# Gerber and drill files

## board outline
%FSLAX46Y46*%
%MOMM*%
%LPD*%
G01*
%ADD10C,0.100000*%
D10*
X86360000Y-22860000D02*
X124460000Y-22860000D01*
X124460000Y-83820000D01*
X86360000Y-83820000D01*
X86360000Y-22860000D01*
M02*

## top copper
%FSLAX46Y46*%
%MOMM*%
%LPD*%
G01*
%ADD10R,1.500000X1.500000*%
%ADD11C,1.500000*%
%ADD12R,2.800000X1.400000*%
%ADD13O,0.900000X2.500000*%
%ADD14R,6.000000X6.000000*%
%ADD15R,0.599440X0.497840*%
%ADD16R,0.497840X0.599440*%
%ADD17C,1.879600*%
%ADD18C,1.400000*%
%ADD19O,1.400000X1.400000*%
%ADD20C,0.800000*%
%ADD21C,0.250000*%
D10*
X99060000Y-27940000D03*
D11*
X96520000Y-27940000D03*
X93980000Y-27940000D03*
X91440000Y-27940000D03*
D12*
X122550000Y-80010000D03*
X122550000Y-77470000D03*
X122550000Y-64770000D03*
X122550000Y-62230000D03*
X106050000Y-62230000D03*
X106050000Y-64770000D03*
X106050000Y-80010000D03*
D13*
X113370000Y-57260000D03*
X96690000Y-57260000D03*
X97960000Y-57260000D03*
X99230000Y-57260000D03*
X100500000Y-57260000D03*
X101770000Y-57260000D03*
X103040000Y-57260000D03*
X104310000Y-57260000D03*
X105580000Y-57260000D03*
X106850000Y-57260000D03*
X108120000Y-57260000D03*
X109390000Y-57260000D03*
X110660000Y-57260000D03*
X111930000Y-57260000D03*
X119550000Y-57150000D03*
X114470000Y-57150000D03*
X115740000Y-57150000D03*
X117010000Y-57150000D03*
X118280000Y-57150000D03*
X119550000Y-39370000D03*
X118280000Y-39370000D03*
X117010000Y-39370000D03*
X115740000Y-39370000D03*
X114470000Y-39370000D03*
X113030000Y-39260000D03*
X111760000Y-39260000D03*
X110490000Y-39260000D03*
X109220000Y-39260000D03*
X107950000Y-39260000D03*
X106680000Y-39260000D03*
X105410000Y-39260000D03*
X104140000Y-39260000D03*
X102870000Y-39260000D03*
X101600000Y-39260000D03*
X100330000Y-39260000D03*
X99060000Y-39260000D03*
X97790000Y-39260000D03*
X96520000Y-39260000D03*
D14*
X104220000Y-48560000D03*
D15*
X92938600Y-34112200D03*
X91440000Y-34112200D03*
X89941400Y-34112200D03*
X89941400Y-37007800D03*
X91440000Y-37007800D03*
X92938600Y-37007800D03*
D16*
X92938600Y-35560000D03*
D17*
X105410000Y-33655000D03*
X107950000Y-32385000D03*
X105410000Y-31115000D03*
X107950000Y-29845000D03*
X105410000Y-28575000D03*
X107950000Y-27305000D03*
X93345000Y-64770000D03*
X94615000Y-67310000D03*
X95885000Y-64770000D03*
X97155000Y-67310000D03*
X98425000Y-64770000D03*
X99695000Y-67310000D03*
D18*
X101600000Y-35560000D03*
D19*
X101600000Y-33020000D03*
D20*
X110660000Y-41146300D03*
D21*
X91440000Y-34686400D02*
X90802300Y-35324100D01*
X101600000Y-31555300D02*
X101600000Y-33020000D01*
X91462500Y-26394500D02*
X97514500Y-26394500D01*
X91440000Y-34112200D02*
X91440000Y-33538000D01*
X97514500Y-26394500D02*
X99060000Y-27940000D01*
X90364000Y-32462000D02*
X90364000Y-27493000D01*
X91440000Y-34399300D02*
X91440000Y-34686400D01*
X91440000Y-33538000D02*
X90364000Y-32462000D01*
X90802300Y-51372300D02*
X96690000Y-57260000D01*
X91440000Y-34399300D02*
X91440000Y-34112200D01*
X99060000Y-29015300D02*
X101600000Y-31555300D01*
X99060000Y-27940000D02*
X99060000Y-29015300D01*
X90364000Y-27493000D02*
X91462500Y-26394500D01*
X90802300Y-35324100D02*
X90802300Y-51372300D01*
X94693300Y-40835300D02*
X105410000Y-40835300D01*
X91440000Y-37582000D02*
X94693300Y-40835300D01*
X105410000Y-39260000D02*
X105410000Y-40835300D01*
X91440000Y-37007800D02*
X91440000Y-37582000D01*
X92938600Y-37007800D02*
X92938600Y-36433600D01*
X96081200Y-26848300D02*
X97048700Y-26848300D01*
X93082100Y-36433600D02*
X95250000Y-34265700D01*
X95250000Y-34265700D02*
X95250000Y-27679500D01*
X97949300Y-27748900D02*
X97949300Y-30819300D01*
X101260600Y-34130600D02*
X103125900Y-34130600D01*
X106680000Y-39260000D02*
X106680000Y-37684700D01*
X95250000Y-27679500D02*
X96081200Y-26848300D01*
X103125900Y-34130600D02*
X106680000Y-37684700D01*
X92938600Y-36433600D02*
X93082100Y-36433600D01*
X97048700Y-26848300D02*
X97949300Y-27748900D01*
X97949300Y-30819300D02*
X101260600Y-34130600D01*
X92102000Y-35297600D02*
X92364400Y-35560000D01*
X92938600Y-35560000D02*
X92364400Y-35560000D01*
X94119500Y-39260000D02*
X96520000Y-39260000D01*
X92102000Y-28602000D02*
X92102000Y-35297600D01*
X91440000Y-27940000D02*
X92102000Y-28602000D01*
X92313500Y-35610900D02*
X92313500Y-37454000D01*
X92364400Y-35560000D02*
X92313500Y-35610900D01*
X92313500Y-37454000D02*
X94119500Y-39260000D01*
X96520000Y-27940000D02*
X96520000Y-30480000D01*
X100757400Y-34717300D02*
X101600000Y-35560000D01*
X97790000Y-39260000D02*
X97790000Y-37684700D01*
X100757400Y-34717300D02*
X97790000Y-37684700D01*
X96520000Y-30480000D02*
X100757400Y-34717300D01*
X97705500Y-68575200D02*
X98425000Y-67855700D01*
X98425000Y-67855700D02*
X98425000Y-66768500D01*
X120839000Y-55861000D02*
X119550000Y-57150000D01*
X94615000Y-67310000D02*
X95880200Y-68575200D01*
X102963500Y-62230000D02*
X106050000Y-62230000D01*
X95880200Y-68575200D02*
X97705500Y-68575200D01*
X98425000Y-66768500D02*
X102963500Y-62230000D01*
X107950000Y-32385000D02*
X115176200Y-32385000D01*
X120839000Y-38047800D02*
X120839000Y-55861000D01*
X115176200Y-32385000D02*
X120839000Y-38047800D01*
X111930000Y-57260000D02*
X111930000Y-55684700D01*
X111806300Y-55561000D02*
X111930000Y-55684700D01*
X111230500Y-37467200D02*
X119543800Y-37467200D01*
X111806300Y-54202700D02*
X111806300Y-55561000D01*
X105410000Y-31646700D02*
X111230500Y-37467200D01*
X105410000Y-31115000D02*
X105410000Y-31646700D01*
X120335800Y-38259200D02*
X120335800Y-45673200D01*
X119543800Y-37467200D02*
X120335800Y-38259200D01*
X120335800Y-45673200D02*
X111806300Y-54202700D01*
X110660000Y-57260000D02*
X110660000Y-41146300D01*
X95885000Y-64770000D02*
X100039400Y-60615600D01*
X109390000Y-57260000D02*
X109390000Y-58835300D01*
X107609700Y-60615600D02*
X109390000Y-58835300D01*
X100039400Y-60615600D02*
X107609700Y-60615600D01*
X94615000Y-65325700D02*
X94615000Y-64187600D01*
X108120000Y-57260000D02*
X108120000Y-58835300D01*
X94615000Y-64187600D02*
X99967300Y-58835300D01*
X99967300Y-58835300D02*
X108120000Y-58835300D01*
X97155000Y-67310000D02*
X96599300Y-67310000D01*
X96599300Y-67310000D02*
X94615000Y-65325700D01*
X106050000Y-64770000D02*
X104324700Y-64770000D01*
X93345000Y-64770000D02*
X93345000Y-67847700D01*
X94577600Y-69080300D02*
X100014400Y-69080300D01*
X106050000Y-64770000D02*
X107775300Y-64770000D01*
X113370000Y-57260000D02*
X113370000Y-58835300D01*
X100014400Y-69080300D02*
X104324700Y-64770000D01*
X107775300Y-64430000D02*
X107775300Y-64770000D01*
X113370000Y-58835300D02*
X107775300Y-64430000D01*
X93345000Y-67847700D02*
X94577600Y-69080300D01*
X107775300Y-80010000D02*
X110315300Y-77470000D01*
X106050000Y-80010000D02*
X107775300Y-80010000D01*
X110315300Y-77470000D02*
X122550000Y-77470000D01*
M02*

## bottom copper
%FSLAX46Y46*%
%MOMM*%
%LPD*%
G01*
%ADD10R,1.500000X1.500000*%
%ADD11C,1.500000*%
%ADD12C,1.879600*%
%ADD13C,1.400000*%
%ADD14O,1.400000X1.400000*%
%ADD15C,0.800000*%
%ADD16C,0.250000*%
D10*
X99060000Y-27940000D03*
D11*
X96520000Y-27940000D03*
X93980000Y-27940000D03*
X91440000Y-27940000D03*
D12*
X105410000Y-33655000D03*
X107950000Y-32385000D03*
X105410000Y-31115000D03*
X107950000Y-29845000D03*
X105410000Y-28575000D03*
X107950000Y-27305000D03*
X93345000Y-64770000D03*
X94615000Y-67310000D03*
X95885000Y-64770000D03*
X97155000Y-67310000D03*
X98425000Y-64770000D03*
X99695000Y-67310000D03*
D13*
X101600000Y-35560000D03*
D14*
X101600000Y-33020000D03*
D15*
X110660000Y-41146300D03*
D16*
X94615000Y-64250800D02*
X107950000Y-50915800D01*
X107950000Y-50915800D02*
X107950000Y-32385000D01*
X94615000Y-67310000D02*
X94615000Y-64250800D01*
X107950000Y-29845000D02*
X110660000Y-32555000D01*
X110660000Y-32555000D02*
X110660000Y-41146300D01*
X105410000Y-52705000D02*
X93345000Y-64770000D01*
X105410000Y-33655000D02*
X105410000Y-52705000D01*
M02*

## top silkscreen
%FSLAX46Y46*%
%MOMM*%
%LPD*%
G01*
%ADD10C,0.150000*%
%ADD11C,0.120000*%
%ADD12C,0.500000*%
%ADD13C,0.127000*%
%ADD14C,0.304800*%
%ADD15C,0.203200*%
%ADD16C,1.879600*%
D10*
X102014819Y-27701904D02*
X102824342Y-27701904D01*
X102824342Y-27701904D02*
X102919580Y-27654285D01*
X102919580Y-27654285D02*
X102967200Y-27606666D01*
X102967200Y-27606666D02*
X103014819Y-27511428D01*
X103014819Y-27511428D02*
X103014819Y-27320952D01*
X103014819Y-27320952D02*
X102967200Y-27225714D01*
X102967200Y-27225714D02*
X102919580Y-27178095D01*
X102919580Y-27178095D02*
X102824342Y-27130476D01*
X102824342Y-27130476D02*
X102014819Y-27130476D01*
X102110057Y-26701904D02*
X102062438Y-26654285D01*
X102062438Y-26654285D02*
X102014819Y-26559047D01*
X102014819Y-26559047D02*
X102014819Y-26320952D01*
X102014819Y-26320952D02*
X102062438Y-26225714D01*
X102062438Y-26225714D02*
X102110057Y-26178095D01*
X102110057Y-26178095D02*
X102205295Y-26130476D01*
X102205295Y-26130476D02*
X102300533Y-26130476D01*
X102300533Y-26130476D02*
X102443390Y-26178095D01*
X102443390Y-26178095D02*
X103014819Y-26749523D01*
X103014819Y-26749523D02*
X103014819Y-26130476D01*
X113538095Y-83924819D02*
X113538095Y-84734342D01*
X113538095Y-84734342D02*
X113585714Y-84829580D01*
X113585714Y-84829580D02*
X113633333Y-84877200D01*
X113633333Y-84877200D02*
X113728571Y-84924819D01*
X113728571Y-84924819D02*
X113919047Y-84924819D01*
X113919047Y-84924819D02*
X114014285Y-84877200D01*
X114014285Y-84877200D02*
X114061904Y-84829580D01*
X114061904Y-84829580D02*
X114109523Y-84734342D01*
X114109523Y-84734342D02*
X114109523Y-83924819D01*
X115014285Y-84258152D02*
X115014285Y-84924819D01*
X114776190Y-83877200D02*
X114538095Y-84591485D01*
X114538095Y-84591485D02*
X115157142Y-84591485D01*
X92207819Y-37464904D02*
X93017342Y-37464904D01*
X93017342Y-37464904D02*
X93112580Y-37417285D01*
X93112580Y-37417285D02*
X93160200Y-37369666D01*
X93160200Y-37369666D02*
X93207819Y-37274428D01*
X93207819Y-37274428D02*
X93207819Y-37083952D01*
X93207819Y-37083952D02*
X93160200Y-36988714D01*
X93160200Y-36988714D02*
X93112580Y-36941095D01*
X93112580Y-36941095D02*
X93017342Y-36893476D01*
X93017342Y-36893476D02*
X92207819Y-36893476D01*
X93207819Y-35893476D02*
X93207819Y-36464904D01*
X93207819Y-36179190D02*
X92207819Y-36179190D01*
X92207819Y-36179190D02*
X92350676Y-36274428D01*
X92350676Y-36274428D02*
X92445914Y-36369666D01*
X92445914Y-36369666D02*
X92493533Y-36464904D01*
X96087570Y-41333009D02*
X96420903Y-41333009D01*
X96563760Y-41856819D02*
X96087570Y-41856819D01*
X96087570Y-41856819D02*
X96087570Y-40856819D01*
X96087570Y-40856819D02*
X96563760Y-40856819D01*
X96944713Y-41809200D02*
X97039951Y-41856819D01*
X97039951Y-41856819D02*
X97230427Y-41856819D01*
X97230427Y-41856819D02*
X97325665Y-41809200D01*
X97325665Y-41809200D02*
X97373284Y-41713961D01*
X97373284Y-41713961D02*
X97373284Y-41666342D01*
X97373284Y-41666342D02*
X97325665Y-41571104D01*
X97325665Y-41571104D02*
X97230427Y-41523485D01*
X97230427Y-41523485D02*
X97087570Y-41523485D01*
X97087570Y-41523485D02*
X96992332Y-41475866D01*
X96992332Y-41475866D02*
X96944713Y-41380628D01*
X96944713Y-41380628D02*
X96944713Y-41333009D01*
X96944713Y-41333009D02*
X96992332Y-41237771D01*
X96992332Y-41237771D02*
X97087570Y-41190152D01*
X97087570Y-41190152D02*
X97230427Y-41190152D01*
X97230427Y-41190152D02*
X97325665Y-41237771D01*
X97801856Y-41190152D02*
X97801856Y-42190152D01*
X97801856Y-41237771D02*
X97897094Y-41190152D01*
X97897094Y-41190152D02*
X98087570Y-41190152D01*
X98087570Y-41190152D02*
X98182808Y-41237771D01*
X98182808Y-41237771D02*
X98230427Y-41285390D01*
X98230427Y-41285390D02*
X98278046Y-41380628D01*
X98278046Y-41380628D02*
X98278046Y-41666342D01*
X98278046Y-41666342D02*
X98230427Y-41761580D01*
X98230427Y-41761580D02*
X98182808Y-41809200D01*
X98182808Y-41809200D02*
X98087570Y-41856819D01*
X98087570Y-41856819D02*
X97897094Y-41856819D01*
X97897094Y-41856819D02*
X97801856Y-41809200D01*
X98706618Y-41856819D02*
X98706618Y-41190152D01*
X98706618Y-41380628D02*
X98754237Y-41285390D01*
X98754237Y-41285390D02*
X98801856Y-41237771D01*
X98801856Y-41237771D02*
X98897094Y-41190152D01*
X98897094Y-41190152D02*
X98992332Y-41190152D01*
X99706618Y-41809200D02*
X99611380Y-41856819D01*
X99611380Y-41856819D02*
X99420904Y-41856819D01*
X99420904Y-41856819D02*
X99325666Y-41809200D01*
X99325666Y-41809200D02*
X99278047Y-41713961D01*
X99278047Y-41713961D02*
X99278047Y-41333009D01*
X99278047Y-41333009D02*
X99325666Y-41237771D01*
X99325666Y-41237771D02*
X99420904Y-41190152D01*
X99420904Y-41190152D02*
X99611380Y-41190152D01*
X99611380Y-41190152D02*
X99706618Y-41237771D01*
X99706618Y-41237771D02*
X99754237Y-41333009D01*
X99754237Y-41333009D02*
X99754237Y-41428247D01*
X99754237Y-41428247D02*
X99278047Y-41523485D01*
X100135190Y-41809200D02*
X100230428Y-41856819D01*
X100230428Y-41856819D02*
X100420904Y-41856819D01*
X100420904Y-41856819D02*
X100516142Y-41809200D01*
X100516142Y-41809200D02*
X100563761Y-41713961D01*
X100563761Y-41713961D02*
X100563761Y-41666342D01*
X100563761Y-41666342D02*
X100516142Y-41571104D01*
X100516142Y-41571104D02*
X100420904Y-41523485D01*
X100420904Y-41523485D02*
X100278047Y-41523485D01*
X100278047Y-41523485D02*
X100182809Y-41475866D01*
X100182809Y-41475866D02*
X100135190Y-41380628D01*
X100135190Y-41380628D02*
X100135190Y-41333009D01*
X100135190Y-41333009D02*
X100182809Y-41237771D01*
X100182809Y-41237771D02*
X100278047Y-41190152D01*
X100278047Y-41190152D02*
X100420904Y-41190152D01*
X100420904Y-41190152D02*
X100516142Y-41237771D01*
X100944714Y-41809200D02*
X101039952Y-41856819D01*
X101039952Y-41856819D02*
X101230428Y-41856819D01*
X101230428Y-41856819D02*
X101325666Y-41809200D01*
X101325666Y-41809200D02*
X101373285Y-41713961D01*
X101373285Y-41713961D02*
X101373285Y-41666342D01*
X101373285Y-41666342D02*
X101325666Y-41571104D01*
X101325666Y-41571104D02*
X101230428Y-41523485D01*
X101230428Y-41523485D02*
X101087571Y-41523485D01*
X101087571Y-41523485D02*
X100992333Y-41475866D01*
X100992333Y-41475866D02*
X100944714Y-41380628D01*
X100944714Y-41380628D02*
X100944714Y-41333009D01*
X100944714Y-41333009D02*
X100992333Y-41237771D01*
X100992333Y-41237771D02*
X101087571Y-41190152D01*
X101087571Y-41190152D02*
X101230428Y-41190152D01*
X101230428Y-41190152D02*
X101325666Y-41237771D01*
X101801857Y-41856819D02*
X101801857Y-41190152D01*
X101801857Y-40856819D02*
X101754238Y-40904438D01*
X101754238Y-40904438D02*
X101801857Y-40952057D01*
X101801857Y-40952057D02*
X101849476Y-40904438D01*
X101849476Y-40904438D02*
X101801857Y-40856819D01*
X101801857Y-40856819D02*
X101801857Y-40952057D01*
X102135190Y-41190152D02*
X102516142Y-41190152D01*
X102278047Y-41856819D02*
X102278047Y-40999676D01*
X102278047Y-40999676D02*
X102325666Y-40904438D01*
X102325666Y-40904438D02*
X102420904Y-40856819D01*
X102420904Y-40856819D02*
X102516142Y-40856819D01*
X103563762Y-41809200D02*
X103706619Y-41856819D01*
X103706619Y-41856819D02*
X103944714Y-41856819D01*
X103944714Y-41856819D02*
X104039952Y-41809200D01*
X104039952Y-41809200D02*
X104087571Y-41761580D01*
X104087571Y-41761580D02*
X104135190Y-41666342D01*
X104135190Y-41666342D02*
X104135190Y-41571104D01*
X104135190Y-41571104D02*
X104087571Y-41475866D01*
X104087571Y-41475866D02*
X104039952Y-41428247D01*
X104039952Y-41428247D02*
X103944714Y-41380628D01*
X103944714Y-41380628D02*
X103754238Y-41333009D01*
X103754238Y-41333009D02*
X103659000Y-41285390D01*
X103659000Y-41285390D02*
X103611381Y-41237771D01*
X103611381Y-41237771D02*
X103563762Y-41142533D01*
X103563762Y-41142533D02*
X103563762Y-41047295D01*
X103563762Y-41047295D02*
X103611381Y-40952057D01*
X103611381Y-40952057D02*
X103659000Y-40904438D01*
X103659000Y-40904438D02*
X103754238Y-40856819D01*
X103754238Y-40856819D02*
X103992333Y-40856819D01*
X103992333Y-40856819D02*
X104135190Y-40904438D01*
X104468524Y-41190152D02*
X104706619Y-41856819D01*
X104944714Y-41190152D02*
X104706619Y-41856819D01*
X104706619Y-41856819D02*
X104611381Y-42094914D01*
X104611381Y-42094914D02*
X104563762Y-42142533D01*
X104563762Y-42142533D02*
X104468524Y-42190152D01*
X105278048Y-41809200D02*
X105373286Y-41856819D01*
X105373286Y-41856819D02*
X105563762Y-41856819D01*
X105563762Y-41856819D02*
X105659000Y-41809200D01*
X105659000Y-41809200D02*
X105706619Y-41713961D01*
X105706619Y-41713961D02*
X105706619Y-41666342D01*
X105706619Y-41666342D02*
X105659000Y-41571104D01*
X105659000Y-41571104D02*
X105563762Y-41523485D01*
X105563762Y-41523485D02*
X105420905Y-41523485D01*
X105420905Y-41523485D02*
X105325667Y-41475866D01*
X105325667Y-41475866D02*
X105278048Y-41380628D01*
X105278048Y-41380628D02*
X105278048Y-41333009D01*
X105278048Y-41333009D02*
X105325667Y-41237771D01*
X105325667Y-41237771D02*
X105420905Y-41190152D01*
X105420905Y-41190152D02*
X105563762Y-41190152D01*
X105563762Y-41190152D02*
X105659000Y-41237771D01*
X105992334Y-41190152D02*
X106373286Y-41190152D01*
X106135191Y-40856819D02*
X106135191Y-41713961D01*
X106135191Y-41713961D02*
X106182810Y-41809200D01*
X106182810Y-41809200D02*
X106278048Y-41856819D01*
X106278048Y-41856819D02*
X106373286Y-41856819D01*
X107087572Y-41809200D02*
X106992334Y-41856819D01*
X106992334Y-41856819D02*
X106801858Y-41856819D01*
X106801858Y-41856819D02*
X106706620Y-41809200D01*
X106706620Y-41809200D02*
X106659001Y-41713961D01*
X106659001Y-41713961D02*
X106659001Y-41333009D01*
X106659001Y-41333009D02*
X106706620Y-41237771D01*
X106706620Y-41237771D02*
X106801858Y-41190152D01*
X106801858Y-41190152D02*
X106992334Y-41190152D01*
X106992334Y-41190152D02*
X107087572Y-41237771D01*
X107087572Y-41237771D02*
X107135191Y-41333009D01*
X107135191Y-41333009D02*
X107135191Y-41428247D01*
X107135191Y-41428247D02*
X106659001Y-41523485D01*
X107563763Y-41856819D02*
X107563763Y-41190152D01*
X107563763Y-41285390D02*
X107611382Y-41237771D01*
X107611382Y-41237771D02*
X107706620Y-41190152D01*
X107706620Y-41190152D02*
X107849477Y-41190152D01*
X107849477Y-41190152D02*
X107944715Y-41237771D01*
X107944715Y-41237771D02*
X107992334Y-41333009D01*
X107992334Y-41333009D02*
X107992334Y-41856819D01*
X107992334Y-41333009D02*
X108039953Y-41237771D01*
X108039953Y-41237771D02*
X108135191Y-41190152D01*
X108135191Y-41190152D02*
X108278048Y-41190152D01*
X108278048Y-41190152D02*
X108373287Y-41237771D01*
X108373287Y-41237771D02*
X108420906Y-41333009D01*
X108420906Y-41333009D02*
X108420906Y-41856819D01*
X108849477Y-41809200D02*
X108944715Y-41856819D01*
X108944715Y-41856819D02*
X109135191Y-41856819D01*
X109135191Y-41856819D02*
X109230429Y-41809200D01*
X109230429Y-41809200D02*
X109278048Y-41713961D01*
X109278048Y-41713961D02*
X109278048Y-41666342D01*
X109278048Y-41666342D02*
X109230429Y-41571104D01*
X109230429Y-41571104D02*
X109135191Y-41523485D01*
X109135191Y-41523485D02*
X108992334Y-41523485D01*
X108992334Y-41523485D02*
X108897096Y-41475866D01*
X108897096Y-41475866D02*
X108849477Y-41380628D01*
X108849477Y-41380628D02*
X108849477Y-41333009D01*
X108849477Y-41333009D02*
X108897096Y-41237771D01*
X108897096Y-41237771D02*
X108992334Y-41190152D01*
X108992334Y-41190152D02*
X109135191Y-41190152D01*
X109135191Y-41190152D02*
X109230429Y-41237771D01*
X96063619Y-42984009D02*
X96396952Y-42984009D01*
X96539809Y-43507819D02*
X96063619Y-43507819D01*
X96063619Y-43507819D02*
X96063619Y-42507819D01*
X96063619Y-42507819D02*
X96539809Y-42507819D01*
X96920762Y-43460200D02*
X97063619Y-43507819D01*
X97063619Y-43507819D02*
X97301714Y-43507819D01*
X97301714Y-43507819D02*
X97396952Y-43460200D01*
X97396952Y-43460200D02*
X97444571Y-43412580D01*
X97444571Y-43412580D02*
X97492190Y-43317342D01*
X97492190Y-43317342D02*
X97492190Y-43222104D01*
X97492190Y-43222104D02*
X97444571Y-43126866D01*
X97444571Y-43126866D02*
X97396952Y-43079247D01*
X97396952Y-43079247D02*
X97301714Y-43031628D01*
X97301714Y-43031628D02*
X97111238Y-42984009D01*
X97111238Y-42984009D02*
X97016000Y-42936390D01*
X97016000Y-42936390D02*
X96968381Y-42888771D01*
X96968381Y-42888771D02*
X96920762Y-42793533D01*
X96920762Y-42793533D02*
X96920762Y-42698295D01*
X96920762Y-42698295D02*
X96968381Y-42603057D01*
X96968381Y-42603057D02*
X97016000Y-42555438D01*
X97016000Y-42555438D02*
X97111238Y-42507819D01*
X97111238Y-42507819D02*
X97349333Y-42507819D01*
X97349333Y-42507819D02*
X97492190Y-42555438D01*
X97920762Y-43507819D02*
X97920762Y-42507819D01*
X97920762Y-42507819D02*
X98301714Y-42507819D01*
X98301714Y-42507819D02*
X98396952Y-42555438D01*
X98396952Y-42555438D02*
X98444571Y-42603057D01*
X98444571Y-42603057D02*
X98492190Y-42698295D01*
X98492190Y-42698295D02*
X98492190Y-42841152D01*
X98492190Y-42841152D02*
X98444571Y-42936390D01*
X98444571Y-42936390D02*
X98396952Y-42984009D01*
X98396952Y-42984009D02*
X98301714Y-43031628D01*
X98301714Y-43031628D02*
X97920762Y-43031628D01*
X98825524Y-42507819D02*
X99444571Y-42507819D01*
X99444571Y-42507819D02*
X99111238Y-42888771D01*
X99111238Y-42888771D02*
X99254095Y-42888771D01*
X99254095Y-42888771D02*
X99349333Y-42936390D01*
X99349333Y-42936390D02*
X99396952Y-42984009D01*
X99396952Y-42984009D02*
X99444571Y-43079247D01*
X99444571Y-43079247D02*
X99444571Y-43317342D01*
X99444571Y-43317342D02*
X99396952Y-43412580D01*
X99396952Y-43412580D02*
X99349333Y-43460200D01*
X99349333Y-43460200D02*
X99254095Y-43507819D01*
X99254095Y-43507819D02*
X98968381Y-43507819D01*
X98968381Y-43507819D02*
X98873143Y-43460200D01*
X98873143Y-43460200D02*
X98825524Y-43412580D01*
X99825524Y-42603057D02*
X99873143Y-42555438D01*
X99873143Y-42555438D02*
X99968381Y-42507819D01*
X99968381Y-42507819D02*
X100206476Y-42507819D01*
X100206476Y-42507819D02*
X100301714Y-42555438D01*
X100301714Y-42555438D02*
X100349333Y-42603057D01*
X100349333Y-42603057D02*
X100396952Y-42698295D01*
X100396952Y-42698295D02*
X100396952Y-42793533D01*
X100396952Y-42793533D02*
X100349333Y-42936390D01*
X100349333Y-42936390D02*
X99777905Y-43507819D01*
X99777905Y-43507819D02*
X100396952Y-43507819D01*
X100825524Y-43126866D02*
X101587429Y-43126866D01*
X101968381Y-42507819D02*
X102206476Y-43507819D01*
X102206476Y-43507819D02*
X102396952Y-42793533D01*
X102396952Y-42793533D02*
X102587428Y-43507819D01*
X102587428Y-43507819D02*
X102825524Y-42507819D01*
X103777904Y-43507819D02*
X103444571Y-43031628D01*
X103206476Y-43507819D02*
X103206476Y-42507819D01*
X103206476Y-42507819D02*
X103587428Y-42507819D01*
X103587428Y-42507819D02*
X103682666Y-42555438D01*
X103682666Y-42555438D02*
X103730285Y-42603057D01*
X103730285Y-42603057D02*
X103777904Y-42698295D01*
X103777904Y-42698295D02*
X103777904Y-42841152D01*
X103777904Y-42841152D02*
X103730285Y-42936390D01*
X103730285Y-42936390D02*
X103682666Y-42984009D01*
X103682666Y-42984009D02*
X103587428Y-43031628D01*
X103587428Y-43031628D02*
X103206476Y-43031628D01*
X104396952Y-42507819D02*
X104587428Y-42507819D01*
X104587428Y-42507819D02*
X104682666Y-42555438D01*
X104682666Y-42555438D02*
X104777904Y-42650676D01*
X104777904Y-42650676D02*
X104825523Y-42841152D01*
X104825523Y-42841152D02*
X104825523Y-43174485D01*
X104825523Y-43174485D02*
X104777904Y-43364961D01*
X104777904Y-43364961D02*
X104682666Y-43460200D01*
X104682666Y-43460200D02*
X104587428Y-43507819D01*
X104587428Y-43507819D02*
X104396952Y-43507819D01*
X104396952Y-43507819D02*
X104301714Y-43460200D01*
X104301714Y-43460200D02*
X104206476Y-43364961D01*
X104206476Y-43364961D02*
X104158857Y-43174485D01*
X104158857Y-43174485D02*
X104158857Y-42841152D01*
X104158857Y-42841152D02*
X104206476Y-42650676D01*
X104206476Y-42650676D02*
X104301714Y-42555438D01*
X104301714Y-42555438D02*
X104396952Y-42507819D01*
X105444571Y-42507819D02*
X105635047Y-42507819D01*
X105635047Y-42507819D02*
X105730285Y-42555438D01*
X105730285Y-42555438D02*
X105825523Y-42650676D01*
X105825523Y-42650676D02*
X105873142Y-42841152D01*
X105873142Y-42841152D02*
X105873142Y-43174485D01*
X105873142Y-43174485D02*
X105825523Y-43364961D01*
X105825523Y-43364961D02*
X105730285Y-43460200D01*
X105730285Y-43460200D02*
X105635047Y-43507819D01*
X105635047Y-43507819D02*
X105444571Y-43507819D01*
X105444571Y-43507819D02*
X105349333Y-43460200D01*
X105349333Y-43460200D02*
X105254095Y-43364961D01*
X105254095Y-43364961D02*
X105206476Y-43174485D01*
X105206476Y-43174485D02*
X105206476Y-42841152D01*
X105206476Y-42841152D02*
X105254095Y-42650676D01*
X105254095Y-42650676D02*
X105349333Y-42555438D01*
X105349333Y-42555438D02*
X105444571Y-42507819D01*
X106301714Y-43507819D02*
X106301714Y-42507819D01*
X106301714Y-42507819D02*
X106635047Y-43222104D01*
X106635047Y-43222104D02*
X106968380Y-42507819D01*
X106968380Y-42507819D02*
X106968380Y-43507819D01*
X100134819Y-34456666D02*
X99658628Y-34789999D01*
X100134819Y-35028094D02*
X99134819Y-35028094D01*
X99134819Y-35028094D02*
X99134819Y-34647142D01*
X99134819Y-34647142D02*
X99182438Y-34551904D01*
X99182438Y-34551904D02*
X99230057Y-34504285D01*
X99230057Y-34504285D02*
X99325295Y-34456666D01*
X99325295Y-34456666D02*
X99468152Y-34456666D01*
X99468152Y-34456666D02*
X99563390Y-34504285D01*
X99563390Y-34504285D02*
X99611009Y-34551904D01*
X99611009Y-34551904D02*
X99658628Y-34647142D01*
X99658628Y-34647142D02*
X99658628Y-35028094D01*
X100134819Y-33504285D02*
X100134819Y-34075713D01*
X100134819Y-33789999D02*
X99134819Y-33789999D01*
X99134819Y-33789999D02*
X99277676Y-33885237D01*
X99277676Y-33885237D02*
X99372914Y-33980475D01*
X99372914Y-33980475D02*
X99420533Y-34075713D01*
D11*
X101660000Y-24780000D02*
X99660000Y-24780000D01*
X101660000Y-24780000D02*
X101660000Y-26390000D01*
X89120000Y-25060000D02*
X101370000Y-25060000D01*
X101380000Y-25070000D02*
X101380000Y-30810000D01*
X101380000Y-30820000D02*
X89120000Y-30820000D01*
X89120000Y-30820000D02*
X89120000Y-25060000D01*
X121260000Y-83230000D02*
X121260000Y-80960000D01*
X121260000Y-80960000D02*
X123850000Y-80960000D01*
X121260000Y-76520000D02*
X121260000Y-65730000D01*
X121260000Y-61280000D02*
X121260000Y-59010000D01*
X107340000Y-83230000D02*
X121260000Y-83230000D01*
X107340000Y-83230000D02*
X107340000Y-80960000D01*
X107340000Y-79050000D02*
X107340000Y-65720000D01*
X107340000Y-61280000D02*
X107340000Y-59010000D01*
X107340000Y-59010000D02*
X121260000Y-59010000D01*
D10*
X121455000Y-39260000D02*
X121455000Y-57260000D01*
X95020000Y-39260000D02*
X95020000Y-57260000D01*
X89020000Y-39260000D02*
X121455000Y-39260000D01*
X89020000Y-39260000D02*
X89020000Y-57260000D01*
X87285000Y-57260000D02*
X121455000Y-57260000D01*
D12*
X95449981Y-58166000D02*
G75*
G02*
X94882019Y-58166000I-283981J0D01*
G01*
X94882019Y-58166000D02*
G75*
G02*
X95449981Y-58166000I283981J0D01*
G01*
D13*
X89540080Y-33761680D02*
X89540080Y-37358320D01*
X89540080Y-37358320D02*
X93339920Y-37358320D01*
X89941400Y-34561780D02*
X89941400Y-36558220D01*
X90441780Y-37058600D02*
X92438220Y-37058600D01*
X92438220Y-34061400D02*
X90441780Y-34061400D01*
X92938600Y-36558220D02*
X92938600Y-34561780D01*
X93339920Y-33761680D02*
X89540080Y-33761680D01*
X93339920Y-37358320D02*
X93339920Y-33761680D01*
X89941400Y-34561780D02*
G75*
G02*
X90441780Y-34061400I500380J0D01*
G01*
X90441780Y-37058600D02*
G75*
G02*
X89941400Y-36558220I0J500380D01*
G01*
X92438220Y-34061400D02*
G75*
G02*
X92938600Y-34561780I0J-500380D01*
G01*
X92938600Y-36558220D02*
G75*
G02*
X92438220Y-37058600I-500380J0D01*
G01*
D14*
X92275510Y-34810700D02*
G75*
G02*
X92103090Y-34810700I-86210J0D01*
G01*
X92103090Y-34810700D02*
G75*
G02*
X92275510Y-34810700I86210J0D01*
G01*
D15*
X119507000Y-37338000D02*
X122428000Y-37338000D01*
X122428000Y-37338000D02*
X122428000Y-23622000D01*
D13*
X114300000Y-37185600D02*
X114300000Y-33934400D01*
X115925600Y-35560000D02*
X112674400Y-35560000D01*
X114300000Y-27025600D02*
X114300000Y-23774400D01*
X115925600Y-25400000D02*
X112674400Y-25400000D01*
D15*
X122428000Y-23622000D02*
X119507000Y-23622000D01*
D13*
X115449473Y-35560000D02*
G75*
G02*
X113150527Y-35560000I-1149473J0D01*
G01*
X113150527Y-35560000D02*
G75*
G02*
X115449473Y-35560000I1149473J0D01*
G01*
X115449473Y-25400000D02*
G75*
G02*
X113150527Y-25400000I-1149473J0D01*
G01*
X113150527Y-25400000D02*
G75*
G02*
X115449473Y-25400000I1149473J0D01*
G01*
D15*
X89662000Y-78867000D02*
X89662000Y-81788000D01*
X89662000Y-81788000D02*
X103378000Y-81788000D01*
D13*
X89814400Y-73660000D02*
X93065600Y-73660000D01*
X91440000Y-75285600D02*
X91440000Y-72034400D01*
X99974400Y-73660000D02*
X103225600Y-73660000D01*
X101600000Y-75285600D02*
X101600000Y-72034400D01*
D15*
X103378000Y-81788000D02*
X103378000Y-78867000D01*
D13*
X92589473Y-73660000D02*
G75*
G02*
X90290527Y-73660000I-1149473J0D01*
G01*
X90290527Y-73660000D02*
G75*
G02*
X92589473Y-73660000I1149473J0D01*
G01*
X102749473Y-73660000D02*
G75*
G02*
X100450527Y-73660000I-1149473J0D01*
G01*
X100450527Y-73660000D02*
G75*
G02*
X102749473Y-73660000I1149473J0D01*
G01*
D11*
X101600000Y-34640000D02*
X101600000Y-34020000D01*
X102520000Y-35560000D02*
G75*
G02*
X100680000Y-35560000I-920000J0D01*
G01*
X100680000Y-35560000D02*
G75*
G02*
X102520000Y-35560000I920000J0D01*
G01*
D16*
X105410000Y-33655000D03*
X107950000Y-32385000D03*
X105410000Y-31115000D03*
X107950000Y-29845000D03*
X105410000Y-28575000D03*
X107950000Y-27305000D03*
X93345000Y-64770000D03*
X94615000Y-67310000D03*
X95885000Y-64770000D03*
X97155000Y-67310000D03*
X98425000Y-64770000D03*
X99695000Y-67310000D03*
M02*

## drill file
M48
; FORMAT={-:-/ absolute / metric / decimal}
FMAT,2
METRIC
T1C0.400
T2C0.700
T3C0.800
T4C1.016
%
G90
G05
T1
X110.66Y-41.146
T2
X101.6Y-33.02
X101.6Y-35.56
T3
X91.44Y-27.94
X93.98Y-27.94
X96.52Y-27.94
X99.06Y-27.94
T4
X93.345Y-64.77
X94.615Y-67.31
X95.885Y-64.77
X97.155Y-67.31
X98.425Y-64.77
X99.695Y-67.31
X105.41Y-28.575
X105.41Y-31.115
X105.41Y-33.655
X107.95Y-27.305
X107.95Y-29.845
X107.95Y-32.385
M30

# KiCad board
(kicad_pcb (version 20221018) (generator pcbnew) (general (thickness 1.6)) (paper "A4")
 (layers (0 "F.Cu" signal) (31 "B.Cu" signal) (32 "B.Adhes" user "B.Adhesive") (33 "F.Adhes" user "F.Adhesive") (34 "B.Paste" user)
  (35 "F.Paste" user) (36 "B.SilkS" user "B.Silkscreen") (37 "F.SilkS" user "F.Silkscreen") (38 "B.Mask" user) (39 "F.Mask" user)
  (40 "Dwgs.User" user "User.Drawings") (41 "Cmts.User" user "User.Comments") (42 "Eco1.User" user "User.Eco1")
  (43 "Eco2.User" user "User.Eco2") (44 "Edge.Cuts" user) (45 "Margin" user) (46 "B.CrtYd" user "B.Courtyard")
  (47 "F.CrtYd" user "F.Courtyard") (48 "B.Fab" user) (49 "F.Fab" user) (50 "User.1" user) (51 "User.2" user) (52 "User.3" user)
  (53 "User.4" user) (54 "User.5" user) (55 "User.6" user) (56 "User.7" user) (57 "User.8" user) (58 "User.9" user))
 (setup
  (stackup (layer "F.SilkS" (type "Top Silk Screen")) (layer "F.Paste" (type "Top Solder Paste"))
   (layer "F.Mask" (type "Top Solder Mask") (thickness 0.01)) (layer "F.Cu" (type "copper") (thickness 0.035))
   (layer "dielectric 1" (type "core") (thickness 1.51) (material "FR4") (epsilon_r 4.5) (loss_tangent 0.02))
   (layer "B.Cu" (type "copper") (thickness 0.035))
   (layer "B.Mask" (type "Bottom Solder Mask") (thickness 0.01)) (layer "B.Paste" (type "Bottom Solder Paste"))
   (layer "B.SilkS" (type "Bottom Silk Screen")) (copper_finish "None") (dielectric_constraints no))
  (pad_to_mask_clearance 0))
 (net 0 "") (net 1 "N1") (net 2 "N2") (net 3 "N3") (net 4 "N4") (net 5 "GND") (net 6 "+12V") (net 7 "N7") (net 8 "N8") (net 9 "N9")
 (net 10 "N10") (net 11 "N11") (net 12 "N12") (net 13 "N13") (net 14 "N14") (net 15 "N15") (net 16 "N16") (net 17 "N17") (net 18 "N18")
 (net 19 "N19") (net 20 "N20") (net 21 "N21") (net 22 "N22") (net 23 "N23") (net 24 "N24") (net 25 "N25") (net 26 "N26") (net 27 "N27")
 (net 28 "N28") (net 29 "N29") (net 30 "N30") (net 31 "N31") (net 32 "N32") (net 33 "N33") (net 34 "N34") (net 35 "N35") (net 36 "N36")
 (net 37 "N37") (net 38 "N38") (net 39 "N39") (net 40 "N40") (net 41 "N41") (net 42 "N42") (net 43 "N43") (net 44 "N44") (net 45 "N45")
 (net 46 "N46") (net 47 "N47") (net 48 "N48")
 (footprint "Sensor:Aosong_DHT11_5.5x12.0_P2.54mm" (layer "F.Cu") (at 99.06 27.94 -90)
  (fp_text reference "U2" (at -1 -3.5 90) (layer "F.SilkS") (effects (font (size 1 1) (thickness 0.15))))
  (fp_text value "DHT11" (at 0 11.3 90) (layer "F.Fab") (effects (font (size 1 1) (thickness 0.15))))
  (fp_line (start -3.16 -2.6) (end -3.16 -0.6) (stroke (width 0.12) (type solid)) (layer "F.SilkS"))
  (fp_line (start -3.16 -2.6) (end -1.55 -2.6) (stroke (width 0.12) (type solid)) (layer "F.SilkS"))
  (fp_line (start -2.88 9.94) (end -2.88 -2.31) (stroke (width 0.12) (type solid)) (layer "F.SilkS"))
  (fp_line (start -2.87 -2.32) (end 2.87 -2.32) (stroke (width 0.12) (type solid)) (layer "F.SilkS"))
  (fp_line (start 2.88 -2.32) (end 2.88 9.94) (stroke (width 0.12) (type solid)) (layer "F.SilkS"))
  (fp_line (start 2.88 9.94) (end -2.88 9.94) (stroke (width 0.12) (type solid)) (layer "F.SilkS"))
  (pad "1" thru_hole rect (at 0 0 270) (size 1.5 1.5) (drill 0.8) (layers "*.Cu" "*.Mask") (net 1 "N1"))
  (pad "2" thru_hole circle (at 0 2.54 270) (size 1.5 1.5) (drill 0.8) (layers "*.Cu" "*.Mask") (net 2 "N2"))
  (pad "3" thru_hole circle (at 0 5.08 270) (size 1.5 1.5) (drill 0.8) (layers "*.Cu" "*.Mask") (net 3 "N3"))
  (pad "4" thru_hole circle (at 0 7.62 270) (size 1.5 1.5) (drill 0.8) (layers "*.Cu" "*.Mask") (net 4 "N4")))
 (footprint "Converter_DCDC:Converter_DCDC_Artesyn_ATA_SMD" (layer "F.Cu") (at 114.3 71.12 180)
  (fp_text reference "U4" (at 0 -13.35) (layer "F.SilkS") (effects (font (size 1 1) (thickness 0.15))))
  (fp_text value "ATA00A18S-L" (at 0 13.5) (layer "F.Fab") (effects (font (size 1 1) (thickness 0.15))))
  (fp_line (start -6.96 -12.11) (end -6.96 -9.84) (stroke (width 0.12) (type solid)) (layer "F.SilkS"))
  (fp_line (start -6.96 -9.84) (end -9.55 -9.84) (stroke (width 0.12) (type solid)) (layer "F.SilkS"))
  (fp_line (start -6.96 -5.4) (end -6.96 5.39) (stroke (width 0.12) (type solid)) (layer "F.SilkS"))
  (fp_line (start -6.96 9.84) (end -6.96 12.11) (stroke (width 0.12) (type solid)) (layer "F.SilkS"))
  (fp_line (start 6.96 -12.11) (end -6.96 -12.11) (stroke (width 0.12) (type solid)) (layer "F.SilkS"))
  (fp_line (start 6.96 -12.11) (end 6.96 -9.84) (stroke (width 0.12) (type solid)) (layer "F.SilkS"))
  (fp_line (start 6.96 -7.93) (end 6.96 5.4) (stroke (width 0.12) (type solid)) (layer "F.SilkS"))
  (fp_line (start 6.96 9.84) (end 6.96 12.11) (stroke (width 0.12) (type solid)) (layer "F.SilkS"))
  (fp_line (start 6.96 12.11) (end -6.96 12.11) (stroke (width 0.12) (type solid)) (layer "F.SilkS"))
  (pad "1" smd rect (at -8.25 -8.89 180) (size 2.8 1.4) (layers "F.Cu" "F.Paste" "F.Mask") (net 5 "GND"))
  (pad "2" smd rect (at -8.25 -6.35 180) (size 2.8 1.4) (layers "F.Cu" "F.Paste" "F.Mask") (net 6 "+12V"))
  (pad "7" smd rect (at -8.25 6.35 180) (size 2.8 1.4) (layers "F.Cu" "F.Paste" "F.Mask") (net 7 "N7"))
  (pad "8" smd rect (at -8.25 8.89 180) (size 2.8 1.4) (layers "F.Cu" "F.Paste" "F.Mask") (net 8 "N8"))
  (pad "9" smd rect (at 8.25 8.89 180) (size 2.8 1.4) (layers "F.Cu" "F.Paste" "F.Mask") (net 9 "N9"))
  (pad "10" smd rect (at 8.25 6.35 180) (size 2.8 1.4) (layers "F.Cu" "F.Paste" "F.Mask") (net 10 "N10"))
  (pad "16" smd rect (at 8.25 -8.89 180) (size 2.8 1.4) (layers "F.Cu" "F.Paste" "F.Mask") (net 6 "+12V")))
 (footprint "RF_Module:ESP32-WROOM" (layer "F.Cu") (at 101.77 48.26 -90)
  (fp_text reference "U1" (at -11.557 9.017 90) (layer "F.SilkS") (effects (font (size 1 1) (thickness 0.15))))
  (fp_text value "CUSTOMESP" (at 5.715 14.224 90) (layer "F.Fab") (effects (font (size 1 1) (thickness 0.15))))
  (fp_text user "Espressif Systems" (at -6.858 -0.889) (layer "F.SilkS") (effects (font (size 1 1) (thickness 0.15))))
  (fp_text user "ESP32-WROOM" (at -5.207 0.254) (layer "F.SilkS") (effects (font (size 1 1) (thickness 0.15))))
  (fp_line (start -9 -19.685) (end 9 -19.685) (stroke (width 0.15) (type solid)) (layer "F.SilkS"))
  (fp_line (start -9 6.75) (end 9 6.75) (stroke (width 0.15) (type solid)) (layer "F.SilkS"))
  (fp_line (start -9 12.75) (end -9 -19.685) (stroke (width 0.15) (type solid)) (layer "F.SilkS"))
  (fp_line (start -9 12.75) (end 9 12.75) (stroke (width 0.15) (type solid)) (layer "F.SilkS"))
  (fp_line (start 9 14.485) (end 9 -19.685) (stroke (width 0.15) (type solid)) (layer "F.SilkS"))
  (fp_circle (center 9.906 6.604) (end 10.033 6.858) (stroke (width 0.5) (type solid)) (fill none) (layer "F.SilkS"))
  (pad "1" smd oval (at 9 -11.6 270) (size 2.5 0.9) (layers "F.Cu" "F.Paste" "F.Mask") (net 10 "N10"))
  (pad "2" smd oval (at 9 5.08 270) (size 2.5 0.9) (layers "F.Cu" "F.Paste" "F.Mask") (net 1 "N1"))
  (pad "3" smd oval (at 9 3.81 270) (size 2.5 0.9) (layers "F.Cu" "F.Paste" "F.Mask") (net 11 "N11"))
  (pad "4" smd oval (at 9 2.54 270) (size 2.5 0.9) (layers "F.Cu" "F.Paste" "F.Mask") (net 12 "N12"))
  (pad "5" smd oval (at 9 1.27 270) (size 2.5 0.9) (layers "F.Cu" "F.Paste" "F.Mask") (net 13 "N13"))
  (pad "6" smd oval (at 9 0 270) (size 2.5 0.9) (layers "F.Cu" "F.Paste" "F.Mask") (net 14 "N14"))
  (pad "7" smd oval (at 9 -1.27 270) (size 2.5 0.9) (layers "F.Cu" "F.Paste" "F.Mask") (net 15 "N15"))
  (pad "8" smd oval (at 9 -2.54 270) (size 2.5 0.9) (layers "F.Cu" "F.Paste" "F.Mask") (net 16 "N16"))
  (pad "9" smd oval (at 9 -3.81 270) (size 2.5 0.9) (layers "F.Cu" "F.Paste" "F.Mask") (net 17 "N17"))
  (pad "10" smd oval (at 9 -5.08 270) (size 2.5 0.9) (layers "F.Cu" "F.Paste" "F.Mask") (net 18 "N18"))
  (pad "11" smd oval (at 9 -6.35 270) (size 2.5 0.9) (layers "F.Cu" "F.Paste" "F.Mask") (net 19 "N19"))
  (pad "12" smd oval (at 9 -7.62 270) (size 2.5 0.9) (layers "F.Cu" "F.Paste" "F.Mask") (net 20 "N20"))
  (pad "13" smd oval (at 9 -8.89 270) (size 2.5 0.9) (layers "F.Cu" "F.Paste" "F.Mask") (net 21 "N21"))
  (pad "14" smd oval (at 9 -10.16 270) (size 2.5 0.9) (layers "F.Cu" "F.Paste" "F.Mask") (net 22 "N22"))
  (pad "15" smd oval (at 8.89 -17.78) (size 0.9 2.5) (layers "F.Cu" "F.Paste" "F.Mask") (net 9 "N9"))
  (pad "16" smd oval (at 8.89 -12.7 180) (size 0.9 2.5) (layers "F.Cu" "F.Paste" "F.Mask") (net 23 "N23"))
  (pad "17" smd oval (at 8.89 -13.97 180) (size 0.9 2.5) (layers "F.Cu" "F.Paste" "F.Mask") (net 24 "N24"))
  (pad "18" smd oval (at 8.89 -15.24 180) (size 0.9 2.5) (layers "F.Cu" "F.Paste" "F.Mask") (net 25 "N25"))
  (pad "19" smd oval (at 8.89 -16.51 180) (size 0.9 2.5) (layers "F.Cu" "F.Paste" "F.Mask") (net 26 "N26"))
  (pad "20" smd oval (at -8.89 -17.78) (size 0.9 2.5) (layers "F.Cu" "F.Paste" "F.Mask") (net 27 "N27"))
  (pad "21" smd oval (at -8.89 -16.51) (size 0.9 2.5) (layers "F.Cu" "F.Paste" "F.Mask") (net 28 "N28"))
  (pad "22" smd oval (at -8.89 -15.24) (size 0.9 2.5) (layers "F.Cu" "F.Paste" "F.Mask") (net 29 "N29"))
  (pad "23" smd oval (at -8.89 -13.97) (size 0.9 2.5) (layers "F.Cu" "F.Paste" "F.Mask") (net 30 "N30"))
  (pad "24" smd oval (at -8.89 -12.7) (size 0.9 2.5) (layers "F.Cu" "F.Paste" "F.Mask") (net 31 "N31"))
  (pad "25" smd oval (at -9 -11.26 270) (size 2.5 0.9) (layers "F.Cu" "F.Paste" "F.Mask") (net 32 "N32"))
  (pad "26" smd oval (at -9 -9.99 270) (size 2.5 0.9) (layers "F.Cu" "F.Paste" "F.Mask") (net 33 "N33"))
  (pad "27" smd oval (at -9 -8.72 270) (size 2.5 0.9) (layers "F.Cu" "F.Paste" "F.Mask") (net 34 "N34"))
  (pad "28" smd oval (at -9 -7.45 270) (size 2.5 0.9) (layers "F.Cu" "F.Paste" "F.Mask") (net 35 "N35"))
  (pad "29" smd oval (at -9 -6.18 270) (size 2.5 0.9) (layers "F.Cu" "F.Paste" "F.Mask") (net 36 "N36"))
  (pad "30" smd oval (at -9 -4.91 270) (size 2.5 0.9) (layers "F.Cu" "F.Paste" "F.Mask") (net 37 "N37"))
  (pad "31" smd oval (at -9 -3.64 270) (size 2.5 0.9) (layers "F.Cu" "F.Paste" "F.Mask") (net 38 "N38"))
  (pad "32" smd oval (at -9 -2.37 270) (size 2.5 0.9) (layers "F.Cu" "F.Paste" "F.Mask") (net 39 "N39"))
  (pad "33" smd oval (at -9 -1.1 270) (size 2.5 0.9) (layers "F.Cu" "F.Paste" "F.Mask") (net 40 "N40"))
  (pad "34" smd oval (at -9 0.17 270) (size 2.5 0.9) (layers "F.Cu" "F.Paste" "F.Mask") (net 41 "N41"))
  (pad "35" smd oval (at -9 1.44 270) (size 2.5 0.9) (layers "F.Cu" "F.Paste" "F.Mask") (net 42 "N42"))
  (pad "36" smd oval (at -9 2.71 270) (size 2.5 0.9) (layers "F.Cu" "F.Paste" "F.Mask") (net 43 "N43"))
  (pad "37" smd oval (at -9 3.98 270) (size 2.5 0.9) (layers "F.Cu" "F.Paste" "F.Mask") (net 2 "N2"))
  (pad "38" smd oval (at -9 5.25 270) (size 2.5 0.9) (layers "F.Cu" "F.Paste" "F.Mask") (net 4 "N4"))
  (pad "39" smd rect (at 0.3 -2.45 270) (size 6 6) (layers "F.Cu" "F.Paste" "F.Mask")))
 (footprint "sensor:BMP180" (layer "F.Cu") (at 91.44 35.56)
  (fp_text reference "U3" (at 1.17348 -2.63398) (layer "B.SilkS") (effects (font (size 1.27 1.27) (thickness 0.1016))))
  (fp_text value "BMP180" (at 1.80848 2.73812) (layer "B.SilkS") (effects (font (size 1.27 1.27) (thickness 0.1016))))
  (fp_line (start -1.89992 -1.79832) (end -1.89992 1.79832) (stroke (width 0.127) (type solid)) (layer "F.SilkS"))
  (fp_line (start -1.89992 1.79832) (end 1.89992 1.79832) (stroke (width 0.127) (type solid)) (layer "F.SilkS"))
  (fp_line (start -1.4986 -0.99822) (end -1.4986 0.99822) (stroke (width 0.127) (type solid)) (layer "F.SilkS"))
  (fp_line (start -0.99822 1.4986) (end 0.99822 1.4986) (stroke (width 0.127) (type solid)) (layer "F.SilkS"))
  (fp_line (start 0.99822 -1.4986) (end -0.99822 -1.4986) (stroke (width 0.127) (type solid)) (layer "F.SilkS"))
  (fp_line (start 1.4986 0.99822) (end 1.4986 -0.99822) (stroke (width 0.127) (type solid)) (layer "F.SilkS"))
  (fp_line (start 1.89992 -1.79832) (end -1.89992 -1.79832) (stroke (width 0.127) (type solid)) (layer "F.SilkS"))
  (fp_line (start 1.89992 1.79832) (end 1.89992 -1.79832) (stroke (width 0.127) (type solid)) (layer "F.SilkS"))
  (fp_arc (start -1.4986 -0.99822) (mid -1.352042 -1.352042) (end -0.99822 -1.4986) (stroke (width 0.127) (type solid)) (layer "F.SilkS"))
  (fp_arc (start -0.99822 1.4986) (mid -1.352042 1.352042) (end -1.4986 0.99822) (stroke (width 0.127) (type solid)) (layer "F.SilkS"))
  (fp_arc (start 0.99822 -1.4986) (mid 1.352042 -1.352042) (end 1.4986 -0.99822) (stroke (width 0.127) (type solid)) (layer "F.SilkS"))
  (fp_arc (start 1.4986 0.99822) (mid 1.352042 1.352042) (end 0.99822 1.4986) (stroke (width 0.127) (type solid)) (layer "F.SilkS"))
  (fp_circle (center 0.7493 -0.7493) (end 0.81026 -0.81026) (stroke (width 0.3048) (type solid)) (fill none) (layer "F.SilkS"))
  (pad "1" smd rect (at 1.4986 -1.4478 90) (size 0.49784 0.59944) (layers "F.Cu" "F.Paste" "F.Mask"))
  (pad "2" smd rect (at 0 -1.4478 90) (size 0.49784 0.59944) (layers "F.Cu" "F.Paste" "F.Mask") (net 1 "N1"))
  (pad "3" smd rect (at -1.4986 -1.4478 90) (size 0.49784 0.59944) (layers "F.Cu" "F.Paste" "F.Mask") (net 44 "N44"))
  (pad "4" smd rect (at -1.4986 1.4478 90) (size 0.49784 0.59944) (layers "F.Cu" "F.Paste" "F.Mask"))
  (pad "5" smd rect (at 0 1.4478 90) (size 0.49784 0.59944) (layers "F.Cu" "F.Paste" "F.Mask") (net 38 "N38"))
  (pad "6" smd rect (at 1.4986 1.4478 90) (size 0.49784 0.59944) (layers "F.Cu" "F.Paste" "F.Mask") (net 37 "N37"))
  (pad "7" smd rect (at 1.4986 0 180) (size 0.49784 0.59944) (layers "F.Cu" "F.Paste" "F.Mask") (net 4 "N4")))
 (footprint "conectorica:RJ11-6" (layer "F.Cu") (at 114.3 30.48 90)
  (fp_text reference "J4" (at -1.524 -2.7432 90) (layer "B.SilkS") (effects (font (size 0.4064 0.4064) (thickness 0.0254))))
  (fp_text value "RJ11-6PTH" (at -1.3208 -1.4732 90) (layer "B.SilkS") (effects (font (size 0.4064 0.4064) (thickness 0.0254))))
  (fp_line (start -6.858 5.207) (end -6.858 8.128) (stroke (width 0.2032) (type solid)) (layer "F.SilkS"))
  (fp_line (start -6.858 8.128) (end 6.858 8.128) (stroke (width 0.2032) (type solid)) (layer "F.SilkS"))
  (fp_line (start -6.7056 0) (end -3.4544 0) (stroke (width 0.127) (type solid)) (layer "F.SilkS"))
  (fp_line (start -5.08 1.6256) (end -5.08 -1.6256) (stroke (width 0.127) (type solid)) (layer "F.SilkS"))
  (fp_line (start 3.4544 0) (end 6.7056 0) (stroke (width 0.127) (type solid)) (layer "F.SilkS"))
  (fp_line (start 5.08 1.6256) (end 5.08 -1.6256) (stroke (width 0.127) (type solid)) (layer "F.SilkS"))
  (fp_line (start 6.858 8.128) (end 6.858 5.207) (stroke (width 0.2032) (type solid)) (layer "F.SilkS"))
  (fp_circle (center -5.08 0) (end -5.8928 0.8128) (stroke (width 0.127) (type solid)) (fill none) (layer "F.SilkS"))
  (fp_circle (center 5.08 0) (end 5.8928 0.8128) (stroke (width 0.127) (type solid)) (fill none) (layer "F.SilkS"))
  (pad "1" thru_hole circle (at -3.175 -8.89 90) (size 1.8796 1.8796) (drill 1.016) (layers "F&B.Cu" "F.Paste" "F.SilkS" "F.Mask")
   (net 10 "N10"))
  (pad "2" thru_hole circle (at -1.905 -6.35 90) (size 1.8796 1.8796) (drill 1.016) (layers "F&B.Cu" "F.Paste" "F.SilkS" "F.Mask")
   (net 9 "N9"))
  (pad "3" thru_hole circle (at -0.635 -8.89 90) (size 1.8796 1.8796) (drill 1.016) (layers "F&B.Cu" "F.Paste" "F.SilkS" "F.Mask")
   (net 22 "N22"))
  (pad "4" thru_hole circle (at 0.635 -6.35 90) (size 1.8796 1.8796) (drill 1.016) (layers "F&B.Cu" "F.Paste" "F.SilkS" "F.Mask")
   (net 21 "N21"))
  (pad "5" thru_hole circle (at 1.905 -8.89 90) (size 1.8796 1.8796) (drill 1.016) (layers "F&B.Cu" "F.Paste" "F.SilkS" "F.Mask")
   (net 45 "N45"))
  (pad "6" thru_hole circle (at 3.175 -6.35 90) (size 1.8796 1.8796) (drill 1.016) (layers "F&B.Cu" "F.Paste" "F.SilkS" "F.Mask")
   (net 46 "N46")))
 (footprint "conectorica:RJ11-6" (layer "F.Cu") (at 96.52 73.66)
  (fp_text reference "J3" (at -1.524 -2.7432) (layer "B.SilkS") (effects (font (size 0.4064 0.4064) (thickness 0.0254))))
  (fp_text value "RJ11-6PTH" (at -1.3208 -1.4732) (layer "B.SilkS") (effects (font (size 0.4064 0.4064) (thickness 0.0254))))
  (fp_line (start -6.858 5.207) (end -6.858 8.128) (stroke (width 0.2032) (type solid)) (layer "F.SilkS"))
  (fp_line (start -6.858 8.128) (end 6.858 8.128) (stroke (width 0.2032) (type solid)) (layer "F.SilkS"))
  (fp_line (start -6.7056 0) (end -3.4544 0) (stroke (width 0.127) (type solid)) (layer "F.SilkS"))
  (fp_line (start -5.08 1.6256) (end -5.08 -1.6256) (stroke (width 0.127) (type solid)) (layer "F.SilkS"))
  (fp_line (start 3.4544 0) (end 6.7056 0) (stroke (width 0.127) (type solid)) (layer "F.SilkS"))
  (fp_line (start 5.08 1.6256) (end 5.08 -1.6256) (stroke (width 0.127) (type solid)) (layer "F.SilkS"))
  (fp_line (start 6.858 8.128) (end 6.858 5.207) (stroke (width 0.2032) (type solid)) (layer "F.SilkS"))
  (fp_circle (center -5.08 0) (end -5.8928 0.8128) (stroke (width 0.127) (type solid)) (fill none) (layer "F.SilkS"))
  (fp_circle (center 5.08 0) (end 5.8928 0.8128) (stroke (width 0.127) (type solid)) (fill none) (layer "F.SilkS"))
  (pad "1" thru_hole circle (at -3.175 -8.89) (size 1.8796 1.8796) (drill 1.016) (layers "F&B.Cu" "F.Paste" "F.SilkS" "F.Mask")
   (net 10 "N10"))
  (pad "2" thru_hole circle (at -1.905 -6.35) (size 1.8796 1.8796) (drill 1.016) (layers "F&B.Cu" "F.Paste" "F.SilkS" "F.Mask") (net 9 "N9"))
  (pad "3" thru_hole circle (at -0.635 -8.89) (size 1.8796 1.8796) (drill 1.016) (layers "F&B.Cu" "F.Paste" "F.SilkS" "F.Mask")
   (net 20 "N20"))
  (pad "4" thru_hole circle (at 0.635 -6.35) (size 1.8796 1.8796) (drill 1.016) (layers "F&B.Cu" "F.Paste" "F.SilkS" "F.Mask")
   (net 19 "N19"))
  (pad "5" thru_hole circle (at 1.905 -8.89) (size 1.8796 1.8796) (drill 1.016) (layers "F&B.Cu" "F.Paste" "F.SilkS" "F.Mask")
   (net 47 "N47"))
  (pad "6" thru_hole circle (at 3.175 -6.35) (size 1.8796 1.8796) (drill 1.016) (layers "F&B.Cu" "F.Paste" "F.SilkS" "F.Mask")
   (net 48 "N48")))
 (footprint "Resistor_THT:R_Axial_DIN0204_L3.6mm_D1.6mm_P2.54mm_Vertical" (layer "F.Cu") (at 101.6 35.56 90)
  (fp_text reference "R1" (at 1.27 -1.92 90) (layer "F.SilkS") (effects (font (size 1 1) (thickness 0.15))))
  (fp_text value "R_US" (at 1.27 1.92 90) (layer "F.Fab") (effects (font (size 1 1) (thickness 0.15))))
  (fp_line (start 0.92 0) (end 1.54 0) (stroke (width 0.12) (type solid)) (layer "F.SilkS"))
  (fp_circle (center 0 0) (end 0.92 0) (stroke (width 0.12) (type solid)) (fill none) (layer "F.SilkS"))
  (pad "1" thru_hole circle (at 0 0 90) (size 1.4 1.4) (drill 0.7) (layers "*.Cu" "*.Mask") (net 2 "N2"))
  (pad "2" thru_hole oval (at 2.54 0 90) (size 1.4 1.4) (drill 0.7) (layers "*.Cu" "*.Mask") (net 1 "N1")))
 (gr_rect (start 86.36 22.86) (end 124.46 83.82) (stroke (width 0.1) (type default)) (fill none) (layer "Edge.Cuts"))
 (segment (start 91.44 34.6864) (end 90.8023 35.3241) (width 0.25) (layer "F.Cu") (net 1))
 (segment (start 101.6 31.5553) (end 101.6 33.02) (width 0.25) (layer "F.Cu") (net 1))
 (segment (start 91.4625 26.3945) (end 97.5145 26.3945) (width 0.25) (layer "F.Cu") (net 1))
 (segment (start 91.44 34.1122) (end 91.44 33.538) (width 0.25) (layer "F.Cu") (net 1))
 (segment (start 97.5145 26.3945) (end 99.06 27.94) (width 0.25) (layer "F.Cu") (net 1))
 (segment (start 90.364 32.462) (end 90.364 27.493) (width 0.25) (layer "F.Cu") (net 1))
 (segment (start 91.44 34.3993) (end 91.44 34.6864) (width 0.25) (layer "F.Cu") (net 1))
 (segment (start 91.44 33.538) (end 90.364 32.462) (width 0.25) (layer "F.Cu") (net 1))
 (segment (start 90.8023 51.3723) (end 96.69 57.26) (width 0.25) (layer "F.Cu") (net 1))
 (segment (start 91.44 34.3993) (end 91.44 34.1122) (width 0.25) (layer "F.Cu") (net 1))
 (segment (start 99.06 29.0153) (end 101.6 31.5553) (width 0.25) (layer "F.Cu") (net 1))
 (segment (start 99.06 27.94) (end 99.06 29.0153) (width 0.25) (layer "F.Cu") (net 1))
 (segment (start 90.364 27.493) (end 91.4625 26.3945) (width 0.25) (layer "F.Cu") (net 1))
 (segment (start 90.8023 35.3241) (end 90.8023 51.3723) (width 0.25) (layer "F.Cu") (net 1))
 (segment (start 94.6933 40.8353) (end 105.41 40.8353) (width 0.25) (layer "F.Cu") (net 38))
 (segment (start 91.44 37.582) (end 94.6933 40.8353) (width 0.25) (layer "F.Cu") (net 38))
 (segment (start 105.41 39.26) (end 105.41 40.8353) (width 0.25) (layer "F.Cu") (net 38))
 (segment (start 91.44 37.0078) (end 91.44 37.582) (width 0.25) (layer "F.Cu") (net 38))
 (segment (start 92.9386 37.0078) (end 92.9386 36.4336) (width 0.25) (layer "F.Cu") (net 37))
 (segment (start 96.0812 26.8483) (end 97.0487 26.8483) (width 0.25) (layer "F.Cu") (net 37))
 (segment (start 93.0821 36.4336) (end 95.25 34.2657) (width 0.25) (layer "F.Cu") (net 37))
 (segment (start 95.25 34.2657) (end 95.25 27.6795) (width 0.25) (layer "F.Cu") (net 37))
 (segment (start 97.9493 27.7489) (end 97.9493 30.8193) (width 0.25) (layer "F.Cu") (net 37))
 (segment (start 101.2606 34.1306) (end 103.1259 34.1306) (width 0.25) (layer "F.Cu") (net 37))
 (segment (start 106.68 39.26) (end 106.68 37.6847) (width 0.25) (layer "F.Cu") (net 37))
 (segment (start 95.25 27.6795) (end 96.0812 26.8483) (width 0.25) (layer "F.Cu") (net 37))
 (segment (start 103.1259 34.1306) (end 106.68 37.6847) (width 0.25) (layer "F.Cu") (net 37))
 (segment (start 92.9386 36.4336) (end 93.0821 36.4336) (width 0.25) (layer "F.Cu") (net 37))
 (segment (start 97.0487 26.8483) (end 97.9493 27.7489) (width 0.25) (layer "F.Cu") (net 37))
 (segment (start 97.9493 30.8193) (end 101.2606 34.1306) (width 0.25) (layer "F.Cu") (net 37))
 (segment (start 92.102 35.2976) (end 92.3644 35.56) (width 0.25) (layer "F.Cu") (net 4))
 (segment (start 92.9386 35.56) (end 92.3644 35.56) (width 0.25) (layer "F.Cu") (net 4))
 (segment (start 94.1195 39.26) (end 96.52 39.26) (width 0.25) (layer "F.Cu") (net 4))
 (segment (start 92.102 28.602) (end 92.102 35.2976) (width 0.25) (layer "F.Cu") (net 4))
 (segment (start 91.44 27.94) (end 92.102 28.602) (width 0.25) (layer "F.Cu") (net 4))
 (segment (start 92.3135 35.6109) (end 92.3135 37.454) (width 0.25) (layer "F.Cu") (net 4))
 (segment (start 92.3644 35.56) (end 92.3135 35.6109) (width 0.25) (layer "F.Cu") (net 4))
 (segment (start 92.3135 37.454) (end 94.1195 39.26) (width 0.25) (layer "F.Cu") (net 4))
 (segment (start 96.52 27.94) (end 96.52 30.48) (width 0.25) (layer "F.Cu") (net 2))
 (segment (start 100.7574 34.7173) (end 101.6 35.56) (width 0.25) (layer "F.Cu") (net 2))
 (segment (start 97.79 39.26) (end 97.79 37.6847) (width 0.25) (layer "F.Cu") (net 2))
 (segment (start 100.7574 34.7173) (end 97.79 37.6847) (width 0.25) (layer "F.Cu") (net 2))
 (segment (start 96.52 30.48) (end 100.7574 34.7173) (width 0.25) (layer "F.Cu") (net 2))
 (segment (start 97.7055 68.5752) (end 98.425 67.8557) (width 0.25) (layer "F.Cu") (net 9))
 (segment (start 98.425 67.8557) (end 98.425 66.7685) (width 0.25) (layer "F.Cu") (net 9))
 (segment (start 120.839 55.861) (end 119.55 57.15) (width 0.25) (layer "F.Cu") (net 9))
 (segment (start 94.615 67.31) (end 95.8802 68.5752) (width 0.25) (layer "F.Cu") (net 9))
 (segment (start 102.9635 62.23) (end 106.05 62.23) (width 0.25) (layer "F.Cu") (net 9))
 (segment (start 95.8802 68.5752) (end 97.7055 68.5752) (width 0.25) (layer "F.Cu") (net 9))
 (segment (start 98.425 66.7685) (end 102.9635 62.23) (width 0.25) (layer "F.Cu") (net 9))
 (segment (start 107.95 32.385) (end 115.1762 32.385) (width 0.25) (layer "F.Cu") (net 9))
 (segment (start 120.839 38.0478) (end 120.839 55.861) (width 0.25) (layer "F.Cu") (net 9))
 (segment (start 115.1762 32.385) (end 120.839 38.0478) (width 0.25) (layer "F.Cu") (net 9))
 (segment (start 94.615 64.2508) (end 107.95 50.9158) (width 0.25) (layer "B.Cu") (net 9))
 (segment (start 107.95 50.9158) (end 107.95 32.385) (width 0.25) (layer "B.Cu") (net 9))
 (segment (start 94.615 67.31) (end 94.615 64.2508) (width 0.25) (layer "B.Cu") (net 9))
 (segment (start 111.93 57.26) (end 111.93 55.6847) (width 0.25) (layer "F.Cu") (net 22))
 (segment (start 111.8063 55.561) (end 111.93 55.6847) (width 0.25) (layer "F.Cu") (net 22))
 (segment (start 111.2305 37.4672) (end 119.5438 37.4672) (width 0.25) (layer "F.Cu") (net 22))
 (segment (start 111.8063 54.2027) (end 111.8063 55.561) (width 0.25) (layer "F.Cu") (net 22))
 (segment (start 105.41 31.6467) (end 111.2305 37.4672) (width 0.25) (layer "F.Cu") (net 22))
 (segment (start 105.41 31.115) (end 105.41 31.6467) (width 0.25) (layer "F.Cu") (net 22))
 (segment (start 120.3358 38.2592) (end 120.3358 45.6732) (width 0.25) (layer "F.Cu") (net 22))
 (segment (start 119.5438 37.4672) (end 120.3358 38.2592) (width 0.25) (layer "F.Cu") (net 22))
 (segment (start 120.3358 45.6732) (end 111.8063 54.2027) (width 0.25) (layer "F.Cu") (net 22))
 (segment (start 110.66 57.26) (end 110.66 41.1463) (width 0.25) (layer "F.Cu") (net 21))
 (via (at 110.66 41.1463) (size 0.8) (drill 0.4) (layers "F.Cu" "B.Cu") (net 21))
 (segment (start 107.95 29.845) (end 110.66 32.555) (width 0.25) (layer "B.Cu") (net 21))
 (segment (start 110.66 32.555) (end 110.66 41.1463) (width 0.25) (layer "B.Cu") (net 21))
 (segment (start 95.885 64.77) (end 100.0394 60.6156) (width 0.25) (layer "F.Cu") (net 20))
 (segment (start 109.39 57.26) (end 109.39 58.8353) (width 0.25) (layer "F.Cu") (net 20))
 (segment (start 107.6097 60.6156) (end 109.39 58.8353) (width 0.25) (layer "F.Cu") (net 20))
 (segment (start 100.0394 60.6156) (end 107.6097 60.6156) (width 0.25) (layer "F.Cu") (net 20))
 (segment (start 94.615 65.3257) (end 94.615 64.1876) (width 0.25) (layer "F.Cu") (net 19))
 (segment (start 108.12 57.26) (end 108.12 58.8353) (width 0.25) (layer "F.Cu") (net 19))
 (segment (start 94.615 64.1876) (end 99.9673 58.8353) (width 0.25) (layer "F.Cu") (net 19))
 (segment (start 99.9673 58.8353) (end 108.12 58.8353) (width 0.25) (layer "F.Cu") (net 19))
 (segment (start 97.155 67.31) (end 96.5993 67.31) (width 0.25) (layer "F.Cu") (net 19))
 (segment (start 96.5993 67.31) (end 94.615 65.3257) (width 0.25) (layer "F.Cu") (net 19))
 (segment (start 106.05 64.77) (end 104.3247 64.77) (width 0.25) (layer "F.Cu") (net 10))
 (segment (start 93.345 64.77) (end 93.345 67.8477) (width 0.25) (layer "F.Cu") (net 10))
 (segment (start 94.5776 69.0803) (end 100.0144 69.0803) (width 0.25) (layer "F.Cu") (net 10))
 (segment (start 106.05 64.77) (end 107.7753 64.77) (width 0.25) (layer "F.Cu") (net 10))
 (segment (start 113.37 57.26) (end 113.37 58.8353) (width 0.25) (layer "F.Cu") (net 10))
 (segment (start 100.0144 69.0803) (end 104.3247 64.77) (width 0.25) (layer "F.Cu") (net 10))
 (segment (start 107.7753 64.43) (end 107.7753 64.77) (width 0.25) (layer "F.Cu") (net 10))
 (segment (start 113.37 58.8353) (end 107.7753 64.43) (width 0.25) (layer "F.Cu") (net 10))
 (segment (start 93.345 67.8477) (end 94.5776 69.0803) (width 0.25) (layer "F.Cu") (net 10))
 (segment (start 105.41 52.705) (end 93.345 64.77) (width 0.25) (layer "B.Cu") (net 10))
 (segment (start 105.41 33.655) (end 105.41 52.705) (width 0.25) (layer "B.Cu") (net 10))
 (segment (start 107.7753 80.01) (end 110.3153 77.47) (width 0.25) (layer "F.Cu") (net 6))
 (segment (start 106.05 80.01) (end 107.7753 80.01) (width 0.25) (layer "F.Cu") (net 6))
 (segment (start 110.3153 77.47) (end 122.55 77.47) (width 0.25) (layer "F.Cu") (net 6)))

